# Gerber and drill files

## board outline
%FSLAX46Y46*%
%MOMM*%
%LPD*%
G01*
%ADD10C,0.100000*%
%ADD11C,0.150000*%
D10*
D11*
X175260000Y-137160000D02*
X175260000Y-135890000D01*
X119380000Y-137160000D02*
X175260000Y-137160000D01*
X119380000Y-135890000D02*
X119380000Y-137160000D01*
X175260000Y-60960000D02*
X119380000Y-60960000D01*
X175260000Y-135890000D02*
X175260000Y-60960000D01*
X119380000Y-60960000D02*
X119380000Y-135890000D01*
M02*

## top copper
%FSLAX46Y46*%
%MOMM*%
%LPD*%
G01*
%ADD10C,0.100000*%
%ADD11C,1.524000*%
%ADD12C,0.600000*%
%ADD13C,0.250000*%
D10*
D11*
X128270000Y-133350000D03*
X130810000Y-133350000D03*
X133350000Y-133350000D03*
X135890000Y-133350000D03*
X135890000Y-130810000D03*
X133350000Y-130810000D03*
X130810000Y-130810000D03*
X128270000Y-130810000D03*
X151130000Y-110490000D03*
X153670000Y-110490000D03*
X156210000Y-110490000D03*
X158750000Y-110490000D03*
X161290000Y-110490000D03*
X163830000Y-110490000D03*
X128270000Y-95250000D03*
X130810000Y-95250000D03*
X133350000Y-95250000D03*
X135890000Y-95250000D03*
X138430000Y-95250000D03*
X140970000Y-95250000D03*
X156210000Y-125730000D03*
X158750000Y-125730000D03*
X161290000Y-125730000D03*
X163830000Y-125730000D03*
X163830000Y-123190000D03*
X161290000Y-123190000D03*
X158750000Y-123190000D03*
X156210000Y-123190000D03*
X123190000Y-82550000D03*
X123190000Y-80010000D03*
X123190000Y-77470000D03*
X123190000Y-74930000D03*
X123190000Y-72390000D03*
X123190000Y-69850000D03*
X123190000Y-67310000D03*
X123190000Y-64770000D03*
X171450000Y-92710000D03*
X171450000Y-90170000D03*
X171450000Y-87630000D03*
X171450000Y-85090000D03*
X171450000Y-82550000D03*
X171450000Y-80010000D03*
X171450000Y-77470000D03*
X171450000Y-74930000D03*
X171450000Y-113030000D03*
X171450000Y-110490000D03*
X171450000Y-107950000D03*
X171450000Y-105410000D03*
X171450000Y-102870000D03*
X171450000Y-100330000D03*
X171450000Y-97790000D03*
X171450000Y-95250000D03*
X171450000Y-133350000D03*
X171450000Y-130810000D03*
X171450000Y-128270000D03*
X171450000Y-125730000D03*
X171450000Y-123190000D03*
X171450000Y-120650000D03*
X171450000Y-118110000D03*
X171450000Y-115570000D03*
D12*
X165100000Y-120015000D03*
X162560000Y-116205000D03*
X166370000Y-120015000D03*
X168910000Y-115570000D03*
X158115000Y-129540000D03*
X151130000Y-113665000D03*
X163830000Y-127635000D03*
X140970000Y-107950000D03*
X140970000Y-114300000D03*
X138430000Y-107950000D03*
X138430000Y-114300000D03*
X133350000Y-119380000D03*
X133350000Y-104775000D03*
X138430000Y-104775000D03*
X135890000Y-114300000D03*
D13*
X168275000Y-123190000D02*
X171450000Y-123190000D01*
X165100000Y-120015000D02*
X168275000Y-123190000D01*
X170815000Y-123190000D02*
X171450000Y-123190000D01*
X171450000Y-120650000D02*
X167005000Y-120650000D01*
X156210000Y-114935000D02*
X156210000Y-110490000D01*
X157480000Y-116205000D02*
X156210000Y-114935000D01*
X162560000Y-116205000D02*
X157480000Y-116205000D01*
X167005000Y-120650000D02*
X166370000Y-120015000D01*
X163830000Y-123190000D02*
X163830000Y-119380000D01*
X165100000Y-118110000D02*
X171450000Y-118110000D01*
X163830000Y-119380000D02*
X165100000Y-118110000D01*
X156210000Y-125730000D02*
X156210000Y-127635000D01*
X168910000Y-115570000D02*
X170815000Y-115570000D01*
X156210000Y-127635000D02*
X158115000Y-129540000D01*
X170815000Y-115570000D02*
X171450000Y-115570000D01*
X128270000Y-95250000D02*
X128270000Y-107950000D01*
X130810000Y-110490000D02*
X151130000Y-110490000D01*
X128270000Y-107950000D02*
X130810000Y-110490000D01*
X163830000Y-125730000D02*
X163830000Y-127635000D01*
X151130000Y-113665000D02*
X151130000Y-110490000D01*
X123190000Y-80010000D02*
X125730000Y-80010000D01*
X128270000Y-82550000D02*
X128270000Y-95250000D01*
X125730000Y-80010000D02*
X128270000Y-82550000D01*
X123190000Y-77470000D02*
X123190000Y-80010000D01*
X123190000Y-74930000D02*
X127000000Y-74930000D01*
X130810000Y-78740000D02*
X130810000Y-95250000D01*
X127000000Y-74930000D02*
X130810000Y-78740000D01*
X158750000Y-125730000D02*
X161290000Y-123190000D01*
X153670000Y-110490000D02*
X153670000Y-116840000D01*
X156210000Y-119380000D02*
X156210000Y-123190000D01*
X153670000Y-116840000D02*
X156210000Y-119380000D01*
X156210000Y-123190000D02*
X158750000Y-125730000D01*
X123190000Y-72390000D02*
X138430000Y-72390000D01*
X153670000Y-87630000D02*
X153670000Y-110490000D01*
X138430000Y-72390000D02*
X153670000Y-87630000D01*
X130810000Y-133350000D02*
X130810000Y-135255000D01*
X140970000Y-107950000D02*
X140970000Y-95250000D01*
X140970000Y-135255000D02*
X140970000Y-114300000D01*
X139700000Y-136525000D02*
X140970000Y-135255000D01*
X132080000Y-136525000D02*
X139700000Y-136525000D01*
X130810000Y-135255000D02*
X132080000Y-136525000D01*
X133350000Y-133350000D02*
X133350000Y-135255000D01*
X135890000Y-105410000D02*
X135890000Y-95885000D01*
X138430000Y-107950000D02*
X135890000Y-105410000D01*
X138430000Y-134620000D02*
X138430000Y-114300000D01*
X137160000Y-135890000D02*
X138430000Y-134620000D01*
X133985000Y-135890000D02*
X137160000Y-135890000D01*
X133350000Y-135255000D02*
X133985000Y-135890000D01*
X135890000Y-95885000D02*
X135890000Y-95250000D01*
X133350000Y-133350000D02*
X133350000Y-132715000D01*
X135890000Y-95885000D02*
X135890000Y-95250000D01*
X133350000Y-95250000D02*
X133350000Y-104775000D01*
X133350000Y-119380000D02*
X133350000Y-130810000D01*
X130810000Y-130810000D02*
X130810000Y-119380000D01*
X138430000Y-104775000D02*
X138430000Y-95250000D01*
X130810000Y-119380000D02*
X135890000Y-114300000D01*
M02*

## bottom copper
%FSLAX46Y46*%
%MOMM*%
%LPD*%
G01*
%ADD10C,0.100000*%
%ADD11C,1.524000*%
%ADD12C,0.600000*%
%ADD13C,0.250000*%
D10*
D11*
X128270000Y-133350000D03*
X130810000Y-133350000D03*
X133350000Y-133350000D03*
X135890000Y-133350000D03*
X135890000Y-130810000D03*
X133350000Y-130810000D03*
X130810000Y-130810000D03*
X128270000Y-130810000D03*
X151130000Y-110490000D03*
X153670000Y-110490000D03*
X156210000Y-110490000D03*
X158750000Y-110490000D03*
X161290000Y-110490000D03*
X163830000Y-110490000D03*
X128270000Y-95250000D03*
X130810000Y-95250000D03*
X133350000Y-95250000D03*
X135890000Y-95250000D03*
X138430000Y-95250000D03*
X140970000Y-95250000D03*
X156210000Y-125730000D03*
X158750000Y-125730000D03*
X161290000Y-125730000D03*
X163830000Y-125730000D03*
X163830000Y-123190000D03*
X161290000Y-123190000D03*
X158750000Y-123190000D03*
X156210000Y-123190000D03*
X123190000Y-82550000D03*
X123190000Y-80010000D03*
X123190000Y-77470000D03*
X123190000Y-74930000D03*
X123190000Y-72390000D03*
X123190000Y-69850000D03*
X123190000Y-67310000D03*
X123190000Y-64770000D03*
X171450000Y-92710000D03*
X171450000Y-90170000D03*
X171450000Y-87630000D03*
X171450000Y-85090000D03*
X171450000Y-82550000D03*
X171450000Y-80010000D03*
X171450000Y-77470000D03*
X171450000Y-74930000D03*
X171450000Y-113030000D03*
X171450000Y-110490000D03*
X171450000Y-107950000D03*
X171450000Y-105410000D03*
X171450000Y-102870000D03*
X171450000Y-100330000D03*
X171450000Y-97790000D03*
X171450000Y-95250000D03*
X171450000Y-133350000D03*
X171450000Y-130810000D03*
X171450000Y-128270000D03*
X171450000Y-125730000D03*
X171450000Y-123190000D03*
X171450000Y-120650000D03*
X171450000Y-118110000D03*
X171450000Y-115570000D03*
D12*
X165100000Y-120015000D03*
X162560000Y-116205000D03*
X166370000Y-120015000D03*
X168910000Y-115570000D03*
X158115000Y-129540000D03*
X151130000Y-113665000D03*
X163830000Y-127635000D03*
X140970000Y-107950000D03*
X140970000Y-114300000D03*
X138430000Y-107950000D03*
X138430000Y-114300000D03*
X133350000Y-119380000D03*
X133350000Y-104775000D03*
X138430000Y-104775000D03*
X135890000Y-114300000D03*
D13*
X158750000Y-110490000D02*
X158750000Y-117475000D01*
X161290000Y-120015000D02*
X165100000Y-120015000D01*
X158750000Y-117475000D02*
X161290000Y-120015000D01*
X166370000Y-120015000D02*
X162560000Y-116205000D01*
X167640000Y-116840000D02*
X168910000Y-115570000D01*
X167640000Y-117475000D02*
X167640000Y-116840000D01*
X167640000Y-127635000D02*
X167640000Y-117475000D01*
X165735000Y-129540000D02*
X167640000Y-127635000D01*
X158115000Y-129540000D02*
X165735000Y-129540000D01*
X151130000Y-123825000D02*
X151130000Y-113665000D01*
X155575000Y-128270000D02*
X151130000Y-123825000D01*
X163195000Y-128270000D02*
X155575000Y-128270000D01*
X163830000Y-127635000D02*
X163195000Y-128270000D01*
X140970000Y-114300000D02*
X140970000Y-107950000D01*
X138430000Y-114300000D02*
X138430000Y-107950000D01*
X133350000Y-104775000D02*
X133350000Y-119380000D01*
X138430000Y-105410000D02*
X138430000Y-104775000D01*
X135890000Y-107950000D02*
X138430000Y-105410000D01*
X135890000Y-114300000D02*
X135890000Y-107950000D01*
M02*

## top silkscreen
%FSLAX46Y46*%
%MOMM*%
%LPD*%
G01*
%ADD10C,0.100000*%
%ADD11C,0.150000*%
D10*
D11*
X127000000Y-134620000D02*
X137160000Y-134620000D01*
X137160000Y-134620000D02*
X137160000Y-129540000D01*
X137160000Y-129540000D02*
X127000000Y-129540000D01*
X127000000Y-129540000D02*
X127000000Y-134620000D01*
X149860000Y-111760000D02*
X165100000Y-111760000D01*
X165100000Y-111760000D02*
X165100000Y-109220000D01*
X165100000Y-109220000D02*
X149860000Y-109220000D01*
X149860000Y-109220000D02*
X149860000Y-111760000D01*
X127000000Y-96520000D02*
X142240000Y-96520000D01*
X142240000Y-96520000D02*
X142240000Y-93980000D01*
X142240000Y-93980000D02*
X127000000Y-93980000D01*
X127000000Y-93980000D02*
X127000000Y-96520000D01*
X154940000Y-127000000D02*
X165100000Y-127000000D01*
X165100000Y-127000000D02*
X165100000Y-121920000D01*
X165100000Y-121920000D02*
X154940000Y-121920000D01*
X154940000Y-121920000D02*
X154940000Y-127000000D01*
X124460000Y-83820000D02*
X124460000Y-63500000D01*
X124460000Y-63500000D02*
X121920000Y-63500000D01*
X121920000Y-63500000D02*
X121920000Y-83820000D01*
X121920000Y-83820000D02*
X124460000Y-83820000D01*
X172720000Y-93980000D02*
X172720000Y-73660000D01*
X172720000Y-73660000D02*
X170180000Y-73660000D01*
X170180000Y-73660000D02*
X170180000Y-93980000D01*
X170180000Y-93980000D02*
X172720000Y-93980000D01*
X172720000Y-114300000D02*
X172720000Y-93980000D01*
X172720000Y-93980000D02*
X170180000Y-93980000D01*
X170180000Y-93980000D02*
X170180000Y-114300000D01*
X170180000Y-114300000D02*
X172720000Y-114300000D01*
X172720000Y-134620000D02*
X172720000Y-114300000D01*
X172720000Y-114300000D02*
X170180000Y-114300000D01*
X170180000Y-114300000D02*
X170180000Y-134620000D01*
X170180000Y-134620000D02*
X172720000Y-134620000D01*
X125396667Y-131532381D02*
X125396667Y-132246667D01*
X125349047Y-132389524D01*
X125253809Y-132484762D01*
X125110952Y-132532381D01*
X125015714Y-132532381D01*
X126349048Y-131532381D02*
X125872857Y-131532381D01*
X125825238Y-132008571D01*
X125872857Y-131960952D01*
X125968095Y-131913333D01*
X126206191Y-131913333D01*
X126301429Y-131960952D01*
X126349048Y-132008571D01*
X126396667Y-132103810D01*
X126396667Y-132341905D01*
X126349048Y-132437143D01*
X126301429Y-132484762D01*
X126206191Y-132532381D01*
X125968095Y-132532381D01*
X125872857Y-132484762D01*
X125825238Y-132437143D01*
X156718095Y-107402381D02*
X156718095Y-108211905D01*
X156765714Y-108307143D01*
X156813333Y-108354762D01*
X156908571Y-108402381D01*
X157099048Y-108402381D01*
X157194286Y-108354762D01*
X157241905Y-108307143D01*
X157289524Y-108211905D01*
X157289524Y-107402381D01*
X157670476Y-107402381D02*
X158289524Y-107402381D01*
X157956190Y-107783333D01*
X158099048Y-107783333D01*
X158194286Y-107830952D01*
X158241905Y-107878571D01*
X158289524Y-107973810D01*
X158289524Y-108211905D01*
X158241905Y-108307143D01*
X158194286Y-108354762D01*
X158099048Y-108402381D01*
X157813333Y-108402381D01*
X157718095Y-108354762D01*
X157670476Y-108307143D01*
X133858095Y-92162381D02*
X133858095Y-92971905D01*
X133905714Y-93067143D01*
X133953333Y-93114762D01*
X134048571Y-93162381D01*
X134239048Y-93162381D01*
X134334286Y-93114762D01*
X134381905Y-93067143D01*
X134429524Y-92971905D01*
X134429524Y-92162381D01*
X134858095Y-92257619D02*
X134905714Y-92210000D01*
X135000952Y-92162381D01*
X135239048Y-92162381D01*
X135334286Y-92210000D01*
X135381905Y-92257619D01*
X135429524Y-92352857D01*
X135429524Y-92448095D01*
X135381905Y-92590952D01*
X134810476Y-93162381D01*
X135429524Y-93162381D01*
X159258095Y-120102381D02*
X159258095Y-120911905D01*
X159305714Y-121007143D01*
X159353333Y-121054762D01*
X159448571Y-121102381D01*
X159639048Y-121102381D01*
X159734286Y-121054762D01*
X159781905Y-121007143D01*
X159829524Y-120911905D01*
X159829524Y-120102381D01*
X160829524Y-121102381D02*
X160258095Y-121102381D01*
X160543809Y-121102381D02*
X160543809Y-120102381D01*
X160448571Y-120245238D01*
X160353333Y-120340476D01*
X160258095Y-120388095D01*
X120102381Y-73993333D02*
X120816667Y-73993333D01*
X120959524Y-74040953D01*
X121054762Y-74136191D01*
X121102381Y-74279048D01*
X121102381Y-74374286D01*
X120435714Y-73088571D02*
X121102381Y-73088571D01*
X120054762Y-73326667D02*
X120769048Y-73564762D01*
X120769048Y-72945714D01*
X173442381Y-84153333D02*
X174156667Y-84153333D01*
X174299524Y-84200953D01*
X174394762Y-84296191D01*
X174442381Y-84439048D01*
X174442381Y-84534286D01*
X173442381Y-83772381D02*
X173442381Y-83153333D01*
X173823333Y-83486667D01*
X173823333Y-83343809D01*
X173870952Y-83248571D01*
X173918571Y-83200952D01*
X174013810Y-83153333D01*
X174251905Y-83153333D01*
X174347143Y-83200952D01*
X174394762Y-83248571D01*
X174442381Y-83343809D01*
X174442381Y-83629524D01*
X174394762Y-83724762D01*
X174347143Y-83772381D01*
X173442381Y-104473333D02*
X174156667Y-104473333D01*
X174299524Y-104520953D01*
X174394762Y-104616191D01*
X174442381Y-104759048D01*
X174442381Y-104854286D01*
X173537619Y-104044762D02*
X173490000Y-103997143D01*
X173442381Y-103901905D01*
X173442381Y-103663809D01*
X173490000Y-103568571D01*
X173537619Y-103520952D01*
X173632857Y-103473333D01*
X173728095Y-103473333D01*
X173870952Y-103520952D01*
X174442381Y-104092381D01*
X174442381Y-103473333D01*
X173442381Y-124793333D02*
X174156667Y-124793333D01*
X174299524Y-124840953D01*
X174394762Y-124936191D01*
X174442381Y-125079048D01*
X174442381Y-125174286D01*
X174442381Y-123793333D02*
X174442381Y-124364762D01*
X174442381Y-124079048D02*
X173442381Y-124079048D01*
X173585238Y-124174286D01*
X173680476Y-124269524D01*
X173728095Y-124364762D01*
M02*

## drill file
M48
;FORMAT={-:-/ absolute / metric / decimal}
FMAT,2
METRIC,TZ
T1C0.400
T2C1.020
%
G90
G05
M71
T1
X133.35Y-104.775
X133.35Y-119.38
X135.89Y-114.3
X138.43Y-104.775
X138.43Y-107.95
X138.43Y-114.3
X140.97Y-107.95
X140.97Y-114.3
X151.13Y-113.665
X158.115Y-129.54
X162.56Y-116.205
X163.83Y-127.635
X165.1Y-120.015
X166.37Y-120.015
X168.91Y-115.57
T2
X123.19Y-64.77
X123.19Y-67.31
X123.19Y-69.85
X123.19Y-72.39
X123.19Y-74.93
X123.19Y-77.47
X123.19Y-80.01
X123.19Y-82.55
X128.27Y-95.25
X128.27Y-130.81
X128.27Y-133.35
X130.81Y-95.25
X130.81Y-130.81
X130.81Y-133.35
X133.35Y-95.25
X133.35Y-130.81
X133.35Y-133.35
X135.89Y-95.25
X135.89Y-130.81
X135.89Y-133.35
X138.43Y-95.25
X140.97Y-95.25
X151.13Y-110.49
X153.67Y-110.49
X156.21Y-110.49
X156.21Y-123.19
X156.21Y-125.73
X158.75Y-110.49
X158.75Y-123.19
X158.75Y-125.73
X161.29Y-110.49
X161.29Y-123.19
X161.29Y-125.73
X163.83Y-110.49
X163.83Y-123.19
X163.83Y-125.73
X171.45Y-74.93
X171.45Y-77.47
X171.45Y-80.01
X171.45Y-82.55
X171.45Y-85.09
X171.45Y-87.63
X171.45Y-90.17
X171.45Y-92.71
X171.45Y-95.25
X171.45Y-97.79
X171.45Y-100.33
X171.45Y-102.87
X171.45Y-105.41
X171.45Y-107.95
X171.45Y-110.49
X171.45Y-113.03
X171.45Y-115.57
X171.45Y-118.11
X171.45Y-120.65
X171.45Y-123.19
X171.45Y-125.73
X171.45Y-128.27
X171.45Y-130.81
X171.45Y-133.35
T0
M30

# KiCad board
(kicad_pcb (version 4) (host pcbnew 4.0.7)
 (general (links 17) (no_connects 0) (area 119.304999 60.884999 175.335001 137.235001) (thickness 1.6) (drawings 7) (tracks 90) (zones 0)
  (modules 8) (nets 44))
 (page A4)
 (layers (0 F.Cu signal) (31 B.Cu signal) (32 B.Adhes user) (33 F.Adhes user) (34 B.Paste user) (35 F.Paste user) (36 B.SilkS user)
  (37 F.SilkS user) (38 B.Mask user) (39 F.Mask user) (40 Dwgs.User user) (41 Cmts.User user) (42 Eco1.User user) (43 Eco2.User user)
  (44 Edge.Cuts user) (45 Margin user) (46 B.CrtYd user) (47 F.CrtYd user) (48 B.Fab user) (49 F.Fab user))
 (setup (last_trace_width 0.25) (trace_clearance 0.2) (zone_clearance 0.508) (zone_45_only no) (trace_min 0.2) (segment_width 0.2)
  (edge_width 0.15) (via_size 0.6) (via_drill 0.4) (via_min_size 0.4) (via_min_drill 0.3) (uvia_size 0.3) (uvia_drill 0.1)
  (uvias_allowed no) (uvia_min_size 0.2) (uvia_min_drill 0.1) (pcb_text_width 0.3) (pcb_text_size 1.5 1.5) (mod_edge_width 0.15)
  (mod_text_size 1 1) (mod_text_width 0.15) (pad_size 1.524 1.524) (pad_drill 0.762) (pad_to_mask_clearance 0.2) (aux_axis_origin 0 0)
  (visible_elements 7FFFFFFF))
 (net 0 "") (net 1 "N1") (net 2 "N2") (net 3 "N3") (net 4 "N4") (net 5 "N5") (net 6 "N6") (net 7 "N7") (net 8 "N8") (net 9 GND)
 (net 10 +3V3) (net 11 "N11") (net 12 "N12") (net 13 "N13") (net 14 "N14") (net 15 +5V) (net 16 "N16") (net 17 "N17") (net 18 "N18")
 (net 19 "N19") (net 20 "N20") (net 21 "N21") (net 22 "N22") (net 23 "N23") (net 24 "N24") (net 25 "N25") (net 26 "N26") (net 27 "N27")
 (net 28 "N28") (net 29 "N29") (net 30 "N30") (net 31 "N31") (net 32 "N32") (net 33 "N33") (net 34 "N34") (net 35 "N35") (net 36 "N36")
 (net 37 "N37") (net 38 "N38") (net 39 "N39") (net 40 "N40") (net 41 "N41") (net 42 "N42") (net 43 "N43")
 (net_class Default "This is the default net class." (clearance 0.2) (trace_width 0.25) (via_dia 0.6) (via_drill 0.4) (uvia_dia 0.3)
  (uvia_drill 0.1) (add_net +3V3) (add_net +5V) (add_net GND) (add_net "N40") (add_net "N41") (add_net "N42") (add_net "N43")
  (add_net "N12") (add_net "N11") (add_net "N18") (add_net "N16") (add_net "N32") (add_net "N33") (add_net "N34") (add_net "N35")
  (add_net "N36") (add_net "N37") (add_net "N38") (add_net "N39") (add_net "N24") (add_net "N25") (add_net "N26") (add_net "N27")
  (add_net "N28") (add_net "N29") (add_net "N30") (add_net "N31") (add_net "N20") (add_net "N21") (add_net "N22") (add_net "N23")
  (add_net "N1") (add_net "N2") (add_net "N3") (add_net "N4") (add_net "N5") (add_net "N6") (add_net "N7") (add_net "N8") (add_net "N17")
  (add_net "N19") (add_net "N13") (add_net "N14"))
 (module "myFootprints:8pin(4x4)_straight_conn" (layer F.Cu) (at 132.08 132.08)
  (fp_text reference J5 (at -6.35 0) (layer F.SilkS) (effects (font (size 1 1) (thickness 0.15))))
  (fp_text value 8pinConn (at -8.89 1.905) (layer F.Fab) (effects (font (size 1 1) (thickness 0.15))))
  (fp_line (start -5.08 2.54) (end 5.08 2.54) (layer F.SilkS) (width 0.15))
  (fp_line (start 5.08 2.54) (end 5.08 -2.54) (layer F.SilkS) (width 0.15))
  (fp_line (start 5.08 -2.54) (end -5.08 -2.54) (layer F.SilkS) (width 0.15))
  (fp_line (start -5.08 -2.54) (end -5.08 2.54) (layer F.SilkS) (width 0.15))
  (pad 1 thru_hole circle (at -3.81 1.27) (size 1.524 1.524) (drill 1.02) (layers *.Cu *.Mask) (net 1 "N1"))
  (pad 2 thru_hole circle (at -1.27 1.27) (size 1.524 1.524) (drill 1.02) (layers *.Cu *.Mask) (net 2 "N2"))
  (pad 3 thru_hole circle (at 1.27 1.27) (size 1.524 1.524) (drill 1.02) (layers *.Cu *.Mask) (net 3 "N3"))
  (pad 4 thru_hole circle (at 3.81 1.27) (size 1.524 1.524) (drill 1.02) (layers *.Cu *.Mask) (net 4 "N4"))
  (pad 5 thru_hole circle (at 3.81 -1.27) (size 1.524 1.524) (drill 1.02) (layers *.Cu *.Mask) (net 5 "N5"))
  (pad 6 thru_hole circle (at 1.27 -1.27) (size 1.524 1.524) (drill 1.02) (layers *.Cu *.Mask) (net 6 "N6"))
  (pad 7 thru_hole circle (at -1.27 -1.27) (size 1.524 1.524) (drill 1.02) (layers *.Cu *.Mask) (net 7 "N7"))
  (pad 8 thru_hole circle (at -3.81 -1.27) (size 1.524 1.524) (drill 1.02) (layers *.Cu *.Mask) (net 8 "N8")))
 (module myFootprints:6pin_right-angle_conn (layer F.Cu) (at 157.48 110.49)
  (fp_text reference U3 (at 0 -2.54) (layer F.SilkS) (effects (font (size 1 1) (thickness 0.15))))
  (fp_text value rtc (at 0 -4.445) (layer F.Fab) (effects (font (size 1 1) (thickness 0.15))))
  (fp_line (start -7.62 1.27) (end 7.62 1.27) (layer F.SilkS) (width 0.15))
  (fp_line (start 7.62 1.27) (end 7.62 -1.27) (layer F.SilkS) (width 0.15))
  (fp_line (start 7.62 -1.27) (end -7.62 -1.27) (layer F.SilkS) (width 0.15))
  (fp_line (start -7.62 -1.27) (end -7.62 1.27) (layer F.SilkS) (width 0.15))
  (pad 1 thru_hole circle (at -6.35 0) (size 1.524 1.524) (drill 1.02) (layers *.Cu *.Mask) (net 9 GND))
  (pad 2 thru_hole circle (at -3.81 0) (size 1.524 1.524) (drill 1.02) (layers *.Cu *.Mask) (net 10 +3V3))
  (pad 3 thru_hole circle (at -1.27 0) (size 1.524 1.524) (drill 1.02) (layers *.Cu *.Mask) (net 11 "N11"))
  (pad 4 thru_hole circle (at 1.27 0) (size 1.524 1.524) (drill 1.02) (layers *.Cu *.Mask) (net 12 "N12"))
  (pad 5 thru_hole circle (at 3.81 0) (size 1.524 1.524) (drill 1.02) (layers *.Cu *.Mask) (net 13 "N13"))
  (pad 6 thru_hole circle (at 6.35 0) (size 1.524 1.524) (drill 1.02) (layers *.Cu *.Mask) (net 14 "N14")))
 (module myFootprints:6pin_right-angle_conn (layer F.Cu) (at 134.62 95.25)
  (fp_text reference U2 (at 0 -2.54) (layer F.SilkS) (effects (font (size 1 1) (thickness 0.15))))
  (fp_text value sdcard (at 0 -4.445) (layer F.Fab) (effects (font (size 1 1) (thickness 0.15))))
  (fp_line (start -7.62 1.27) (end 7.62 1.27) (layer F.SilkS) (width 0.15))
  (fp_line (start 7.62 1.27) (end 7.62 -1.27) (layer F.SilkS) (width 0.15))
  (fp_line (start 7.62 -1.27) (end -7.62 -1.27) (layer F.SilkS) (width 0.15))
  (fp_line (start -7.62 -1.27) (end -7.62 1.27) (layer F.SilkS) (width 0.15))
  (pad 1 thru_hole circle (at -6.35 0) (size 1.524 1.524) (drill 1.02) (layers *.Cu *.Mask) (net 9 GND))
  (pad 2 thru_hole circle (at -3.81 0) (size 1.524 1.524) (drill 1.02) (layers *.Cu *.Mask) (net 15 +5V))
  (pad 3 thru_hole circle (at -1.27 0) (size 1.524 1.524) (drill 1.02) (layers *.Cu *.Mask) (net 6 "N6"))
  (pad 4 thru_hole circle (at 1.27 0) (size 1.524 1.524) (drill 1.02) (layers *.Cu *.Mask) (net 3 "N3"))
  (pad 5 thru_hole circle (at 3.81 0) (size 1.524 1.524) (drill 1.02) (layers *.Cu *.Mask) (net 7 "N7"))
  (pad 6 thru_hole circle (at 6.35 0) (size 1.524 1.524) (drill 1.02) (layers *.Cu *.Mask) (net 2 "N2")))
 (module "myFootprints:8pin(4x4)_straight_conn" (layer F.Cu) (at 160.02 124.46)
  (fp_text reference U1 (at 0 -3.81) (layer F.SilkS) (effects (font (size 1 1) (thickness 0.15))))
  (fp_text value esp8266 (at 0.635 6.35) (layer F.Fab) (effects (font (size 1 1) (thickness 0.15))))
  (fp_line (start -5.08 2.54) (end 5.08 2.54) (layer F.SilkS) (width 0.15))
  (fp_line (start 5.08 2.54) (end 5.08 -2.54) (layer F.SilkS) (width 0.15))
  (fp_line (start 5.08 -2.54) (end -5.08 -2.54) (layer F.SilkS) (width 0.15))
  (fp_line (start -5.08 -2.54) (end -5.08 2.54) (layer F.SilkS) (width 0.15))
  (pad 1 thru_hole circle (at -3.81 1.27) (size 1.524 1.524) (drill 1.02) (layers *.Cu *.Mask) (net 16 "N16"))
  (pad 2 thru_hole circle (at -1.27 1.27) (size 1.524 1.524) (drill 1.02) (layers *.Cu *.Mask) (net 10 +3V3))
  (pad 3 thru_hole circle (at 1.27 1.27) (size 1.524 1.524) (drill 1.02) (layers *.Cu *.Mask) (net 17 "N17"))
  (pad 4 thru_hole circle (at 3.81 1.27) (size 1.524 1.524) (drill 1.02) (layers *.Cu *.Mask) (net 9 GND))
  (pad 5 thru_hole circle (at 3.81 -1.27) (size 1.524 1.524) (drill 1.02) (layers *.Cu *.Mask) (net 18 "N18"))
  (pad 6 thru_hole circle (at 1.27 -1.27) (size 1.524 1.524) (drill 1.02) (layers *.Cu *.Mask) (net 10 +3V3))
  (pad 7 thru_hole circle (at -1.27 -1.27) (size 1.524 1.524) (drill 1.02) (layers *.Cu *.Mask) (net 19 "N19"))
  (pad 8 thru_hole circle (at -3.81 -1.27) (size 1.524 1.524) (drill 1.02) (layers *.Cu *.Mask) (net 10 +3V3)))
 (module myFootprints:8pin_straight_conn (layer F.Cu) (at 123.19 73.66 90)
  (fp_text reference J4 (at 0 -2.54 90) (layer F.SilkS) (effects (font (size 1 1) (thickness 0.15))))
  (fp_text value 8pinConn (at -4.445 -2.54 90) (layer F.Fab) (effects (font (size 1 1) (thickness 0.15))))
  (fp_line (start -10.16 1.27) (end 10.16 1.27) (layer F.SilkS) (width 0.15))
  (fp_line (start 10.16 1.27) (end 10.16 -1.27) (layer F.SilkS) (width 0.15))
  (fp_line (start 10.16 -1.27) (end -10.16 -1.27) (layer F.SilkS) (width 0.15))
  (fp_line (start -10.16 -1.27) (end -10.16 1.27) (layer F.SilkS) (width 0.15))
  (pad 1 thru_hole circle (at -8.89 0 90) (size 1.524 1.524) (drill 1.02) (layers *.Cu *.Mask) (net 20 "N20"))
  (pad 2 thru_hole circle (at -6.35 0 90) (size 1.524 1.524) (drill 1.02) (layers *.Cu *.Mask) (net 9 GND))
  (pad 3 thru_hole circle (at -3.81 0 90) (size 1.524 1.524) (drill 1.02) (layers *.Cu *.Mask) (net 9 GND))
  (pad 4 thru_hole circle (at -1.27 0 90) (size 1.524 1.524) (drill 1.02) (layers *.Cu *.Mask) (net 15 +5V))
  (pad 5 thru_hole circle (at 1.27 0 90) (size 1.524 1.524) (drill 1.02) (layers *.Cu *.Mask) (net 10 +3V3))
  (pad 6 thru_hole circle (at 3.81 0 90) (size 1.524 1.524) (drill 1.02) (layers *.Cu *.Mask) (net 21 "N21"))
  (pad 7 thru_hole circle (at 6.35 0 90) (size 1.524 1.524) (drill 1.02) (layers *.Cu *.Mask) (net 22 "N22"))
  (pad 8 thru_hole circle (at 8.89 0 90) (size 1.524 1.524) (drill 1.02) (layers *.Cu *.Mask) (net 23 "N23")))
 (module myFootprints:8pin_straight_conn (layer F.Cu) (at 171.45 83.82 90)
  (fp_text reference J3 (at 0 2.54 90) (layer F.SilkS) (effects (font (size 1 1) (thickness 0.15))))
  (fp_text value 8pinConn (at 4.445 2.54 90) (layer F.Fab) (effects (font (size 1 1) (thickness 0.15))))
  (fp_line (start -10.16 1.27) (end 10.16 1.27) (layer F.SilkS) (width 0.15))
  (fp_line (start 10.16 1.27) (end 10.16 -1.27) (layer F.SilkS) (width 0.15))
  (fp_line (start 10.16 -1.27) (end -10.16 -1.27) (layer F.SilkS) (width 0.15))
  (fp_line (start -10.16 -1.27) (end -10.16 1.27) (layer F.SilkS) (width 0.15))
  (pad 1 thru_hole circle (at -8.89 0 90) (size 1.524 1.524) (drill 1.02) (layers *.Cu *.Mask) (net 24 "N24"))
  (pad 2 thru_hole circle (at -6.35 0 90) (size 1.524 1.524) (drill 1.02) (layers *.Cu *.Mask) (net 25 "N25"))
  (pad 3 thru_hole circle (at -3.81 0 90) (size 1.524 1.524) (drill 1.02) (layers *.Cu *.Mask) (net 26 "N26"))
  (pad 4 thru_hole circle (at -1.27 0 90) (size 1.524 1.524) (drill 1.02) (layers *.Cu *.Mask) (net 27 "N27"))
  (pad 5 thru_hole circle (at 1.27 0 90) (size 1.524 1.524) (drill 1.02) (layers *.Cu *.Mask) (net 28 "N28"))
  (pad 6 thru_hole circle (at 3.81 0 90) (size 1.524 1.524) (drill 1.02) (layers *.Cu *.Mask) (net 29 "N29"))
  (pad 7 thru_hole circle (at 6.35 0 90) (size 1.524 1.524) (drill 1.02) (layers *.Cu *.Mask) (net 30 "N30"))
  (pad 8 thru_hole circle (at 8.89 0 90) (size 1.524 1.524) (drill 1.02) (layers *.Cu *.Mask) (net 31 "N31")))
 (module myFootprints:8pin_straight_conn (layer F.Cu) (at 171.45 104.14 90)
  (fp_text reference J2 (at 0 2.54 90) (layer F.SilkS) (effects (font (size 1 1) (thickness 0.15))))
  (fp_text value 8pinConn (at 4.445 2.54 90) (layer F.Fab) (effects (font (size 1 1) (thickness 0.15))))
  (fp_line (start -10.16 1.27) (end 10.16 1.27) (layer F.SilkS) (width 0.15))
  (fp_line (start 10.16 1.27) (end 10.16 -1.27) (layer F.SilkS) (width 0.15))
  (fp_line (start 10.16 -1.27) (end -10.16 -1.27) (layer F.SilkS) (width 0.15))
  (fp_line (start -10.16 -1.27) (end -10.16 1.27) (layer F.SilkS) (width 0.15))
  (pad 1 thru_hole circle (at -8.89 0 90) (size 1.524 1.524) (drill 1.02) (layers *.Cu *.Mask) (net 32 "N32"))
  (pad 2 thru_hole circle (at -6.35 0 90) (size 1.524 1.524) (drill 1.02) (layers *.Cu *.Mask) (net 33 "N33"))
  (pad 3 thru_hole circle (at -3.81 0 90) (size 1.524 1.524) (drill 1.02) (layers *.Cu *.Mask) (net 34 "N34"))
  (pad 4 thru_hole circle (at -1.27 0 90) (size 1.524 1.524) (drill 1.02) (layers *.Cu *.Mask) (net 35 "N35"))
  (pad 5 thru_hole circle (at 1.27 0 90) (size 1.524 1.524) (drill 1.02) (layers *.Cu *.Mask) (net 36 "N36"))
  (pad 6 thru_hole circle (at 3.81 0 90) (size 1.524 1.524) (drill 1.02) (layers *.Cu *.Mask) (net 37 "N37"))
  (pad 7 thru_hole circle (at 6.35 0 90) (size 1.524 1.524) (drill 1.02) (layers *.Cu *.Mask) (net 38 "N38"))
  (pad 8 thru_hole circle (at 8.89 0 90) (size 1.524 1.524) (drill 1.02) (layers *.Cu *.Mask) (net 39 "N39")))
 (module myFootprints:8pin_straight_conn (layer F.Cu) (at 171.45 124.46 90)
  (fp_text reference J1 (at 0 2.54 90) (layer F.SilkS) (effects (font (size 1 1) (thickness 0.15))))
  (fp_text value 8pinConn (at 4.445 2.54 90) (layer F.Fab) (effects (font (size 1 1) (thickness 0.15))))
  (fp_line (start -10.16 1.27) (end 10.16 1.27) (layer F.SilkS) (width 0.15))
  (fp_line (start 10.16 1.27) (end 10.16 -1.27) (layer F.SilkS) (width 0.15))
  (fp_line (start 10.16 -1.27) (end -10.16 -1.27) (layer F.SilkS) (width 0.15))
  (fp_line (start -10.16 -1.27) (end -10.16 1.27) (layer F.SilkS) (width 0.15))
  (pad 1 thru_hole circle (at -8.89 0 90) (size 1.524 1.524) (drill 1.02) (layers *.Cu *.Mask) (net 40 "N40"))
  (pad 2 thru_hole circle (at -6.35 0 90) (size 1.524 1.524) (drill 1.02) (layers *.Cu *.Mask) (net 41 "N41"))
  (pad 3 thru_hole circle (at -3.81 0 90) (size 1.524 1.524) (drill 1.02) (layers *.Cu *.Mask) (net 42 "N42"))
  (pad 4 thru_hole circle (at -1.27 0 90) (size 1.524 1.524) (drill 1.02) (layers *.Cu *.Mask) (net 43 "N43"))
  (pad 5 thru_hole circle (at 1.27 0 90) (size 1.524 1.524) (drill 1.02) (layers *.Cu *.Mask) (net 12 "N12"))
  (pad 6 thru_hole circle (at 3.81 0 90) (size 1.524 1.524) (drill 1.02) (layers *.Cu *.Mask) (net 11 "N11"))
  (pad 7 thru_hole circle (at 6.35 0 90) (size 1.524 1.524) (drill 1.02) (layers *.Cu *.Mask) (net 18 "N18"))
  (pad 8 thru_hole circle (at 8.89 0 90) (size 1.524 1.524) (drill 1.02) (layers *.Cu *.Mask) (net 16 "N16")))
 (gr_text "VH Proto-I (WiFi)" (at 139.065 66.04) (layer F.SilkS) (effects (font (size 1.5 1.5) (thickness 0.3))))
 (gr_line (start 175.26 137.16) (end 175.26 135.89) (angle 90) (layer Edge.Cuts) (width 0.15))
 (gr_line (start 119.38 137.16) (end 175.26 137.16) (angle 90) (layer Edge.Cuts) (width 0.15))
 (gr_line (start 119.38 135.89) (end 119.38 137.16) (angle 90) (layer Edge.Cuts) (width 0.15))
 (gr_line (start 175.26 60.96) (end 119.38 60.96) (angle 90) (layer Edge.Cuts) (width 0.15))
 (gr_line (start 175.26 135.89) (end 175.26 60.96) (angle 90) (layer Edge.Cuts) (width 0.15))
 (gr_line (start 119.38 60.96) (end 119.38 135.89) (angle 90) (layer Edge.Cuts) (width 0.15))
 (segment (start 158.75 110.49) (end 158.75 117.475) (width 0.25) (layer B.Cu) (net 12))
 (segment (start 168.275 123.19) (end 171.45 123.19) (width 0.25) (layer F.Cu) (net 12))
 (segment (start 165.1 120.015) (end 168.275 123.19) (width 0.25) (layer F.Cu) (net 12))
 (via (at 165.1 120.015) (size 0.6) (drill 0.4) (layers F.Cu B.Cu) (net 12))
 (segment (start 161.29 120.015) (end 165.1 120.015) (width 0.25) (layer B.Cu) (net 12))
 (segment (start 158.75 117.475) (end 161.29 120.015) (width 0.25) (layer B.Cu) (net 12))
 (segment (start 170.815 123.19) (end 171.45 123.19) (width 0.25) (layer F.Cu) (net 12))
 (segment (start 171.45 120.65) (end 167.005 120.65) (width 0.25) (layer F.Cu) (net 11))
 (segment (start 156.21 114.935) (end 156.21 110.49) (width 0.25) (layer F.Cu) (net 11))
 (segment (start 157.48 116.205) (end 156.21 114.935) (width 0.25) (layer F.Cu) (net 11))
 (segment (start 162.56 116.205) (end 157.48 116.205) (width 0.25) (layer F.Cu) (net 11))
 (via (at 162.56 116.205) (size 0.6) (drill 0.4) (layers F.Cu B.Cu) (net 11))
 (segment (start 166.37 120.015) (end 162.56 116.205) (width 0.25) (layer B.Cu) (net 11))
 (via (at 166.37 120.015) (size 0.6) (drill 0.4) (layers F.Cu B.Cu) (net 11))
 (segment (start 167.005 120.65) (end 166.37 120.015) (width 0.25) (layer F.Cu) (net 11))
 (segment (start 163.83 123.19) (end 163.83 119.38) (width 0.25) (layer F.Cu) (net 18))
 (segment (start 165.1 118.11) (end 171.45 118.11) (width 0.25) (layer F.Cu) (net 18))
 (segment (start 163.83 119.38) (end 165.1 118.11) (width 0.25) (layer F.Cu) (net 18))
 (segment (start 156.21 125.73) (end 156.21 127.635) (width 0.25) (layer F.Cu) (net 16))
 (segment (start 168.91 115.57) (end 170.815 115.57) (width 0.25) (layer F.Cu) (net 16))
 (via (at 168.91 115.57) (size 0.6) (drill 0.4) (layers F.Cu B.Cu) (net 16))
 (segment (start 167.64 116.84) (end 168.91 115.57) (width 0.25) (layer B.Cu) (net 16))
 (segment (start 167.64 117.475) (end 167.64 116.84) (width 0.25) (layer B.Cu) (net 16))
 (segment (start 167.64 127.635) (end 167.64 117.475) (width 0.25) (layer B.Cu) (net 16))
 (segment (start 165.735 129.54) (end 167.64 127.635) (width 0.25) (layer B.Cu) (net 16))
 (segment (start 158.115 129.54) (end 165.735 129.54) (width 0.25) (layer B.Cu) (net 16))
 (via (at 158.115 129.54) (size 0.6) (drill 0.4) (layers F.Cu B.Cu) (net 16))
 (segment (start 156.21 127.635) (end 158.115 129.54) (width 0.25) (layer F.Cu) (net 16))
 (segment (start 170.815 115.57) (end 171.45 115.57) (width 0.25) (layer F.Cu) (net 16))
 (segment (start 128.27 95.25) (end 128.27 107.95) (width 0.25) (layer F.Cu) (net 9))
 (segment (start 130.81 110.49) (end 151.13 110.49) (width 0.25) (layer F.Cu) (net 9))
 (segment (start 128.27 107.95) (end 130.81 110.49) (width 0.25) (layer F.Cu) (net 9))
 (segment (start 163.83 125.73) (end 163.83 127.635) (width 0.25) (layer F.Cu) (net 9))
 (segment (start 151.13 113.665) (end 151.13 110.49) (width 0.25) (layer F.Cu) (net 9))
 (via (at 151.13 113.665) (size 0.6) (drill 0.4) (layers F.Cu B.Cu) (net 9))
 (segment (start 151.13 123.825) (end 151.13 113.665) (width 0.25) (layer B.Cu) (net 9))
 (segment (start 155.575 128.27) (end 151.13 123.825) (width 0.25) (layer B.Cu) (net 9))
 (segment (start 163.195 128.27) (end 155.575 128.27) (width 0.25) (layer B.Cu) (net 9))
 (segment (start 163.83 127.635) (end 163.195 128.27) (width 0.25) (layer B.Cu) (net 9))
 (via (at 163.83 127.635) (size 0.6) (drill 0.4) (layers F.Cu B.Cu) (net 9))
 (segment (start 123.19 80.01) (end 125.73 80.01) (width 0.25) (layer F.Cu) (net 9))
 (segment (start 128.27 82.55) (end 128.27 95.25) (width 0.25) (layer F.Cu) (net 9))
 (segment (start 125.73 80.01) (end 128.27 82.55) (width 0.25) (layer F.Cu) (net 9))
 (segment (start 123.19 77.47) (end 123.19 80.01) (width 0.25) (layer F.Cu) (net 9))
 (segment (start 123.19 74.93) (end 127 74.93) (width 0.25) (layer F.Cu) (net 15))
 (segment (start 130.81 78.74) (end 130.81 95.25) (width 0.25) (layer F.Cu) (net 15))
 (segment (start 127 74.93) (end 130.81 78.74) (width 0.25) (layer F.Cu) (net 15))
 (segment (start 158.75 125.73) (end 161.29 123.19) (width 0.25) (layer F.Cu) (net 10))
 (segment (start 153.67 110.49) (end 153.67 116.84) (width 0.25) (layer F.Cu) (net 10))
 (segment (start 156.21 119.38) (end 156.21 123.19) (width 0.25) (layer F.Cu) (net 10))
 (segment (start 153.67 116.84) (end 156.21 119.38) (width 0.25) (layer F.Cu) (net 10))
 (segment (start 156.21 123.19) (end 158.75 125.73) (width 0.25) (layer F.Cu) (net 10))
 (segment (start 123.19 72.39) (end 138.43 72.39) (width 0.25) (layer F.Cu) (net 10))
 (segment (start 153.67 87.63) (end 153.67 110.49) (width 0.25) (layer F.Cu) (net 10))
 (segment (start 138.43 72.39) (end 153.67 87.63) (width 0.25) (layer F.Cu) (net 10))
 (segment (start 130.81 133.35) (end 130.81 135.255) (width 0.25) (layer F.Cu) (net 2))
 (segment (start 140.97 107.95) (end 140.97 95.25) (width 0.25) (layer F.Cu) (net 2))
 (via (at 140.97 107.95) (size 0.6) (drill 0.4) (layers F.Cu B.Cu) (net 2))
 (segment (start 140.97 114.3) (end 140.97 107.95) (width 0.25) (layer B.Cu) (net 2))
 (via (at 140.97 114.3) (size 0.6) (drill 0.4) (layers F.Cu B.Cu) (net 2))
 (segment (start 140.97 135.255) (end 140.97 114.3) (width 0.25) (layer F.Cu) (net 2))
 (segment (start 139.7 136.525) (end 140.97 135.255) (width 0.25) (layer F.Cu) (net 2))
 (segment (start 132.08 136.525) (end 139.7 136.525) (width 0.25) (layer F.Cu) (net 2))
 (segment (start 130.81 135.255) (end 132.08 136.525) (width 0.25) (layer F.Cu) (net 2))
 (segment (start 133.35 133.35) (end 133.35 135.255) (width 0.25) (layer F.Cu) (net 3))
 (segment (start 135.89 105.41) (end 135.89 95.885) (width 0.25) (layer F.Cu) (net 3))
 (segment (start 138.43 107.95) (end 135.89 105.41) (width 0.25) (layer F.Cu) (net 3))
 (via (at 138.43 107.95) (size 0.6) (drill 0.4) (layers F.Cu B.Cu) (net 3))
 (segment (start 138.43 114.3) (end 138.43 107.95) (width 0.25) (layer B.Cu) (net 3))
 (via (at 138.43 114.3) (size 0.6) (drill 0.4) (layers F.Cu B.Cu) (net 3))
 (segment (start 138.43 134.62) (end 138.43 114.3) (width 0.25) (layer F.Cu) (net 3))
 (segment (start 137.16 135.89) (end 138.43 134.62) (width 0.25) (layer F.Cu) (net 3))
 (segment (start 133.985 135.89) (end 137.16 135.89) (width 0.25) (layer F.Cu) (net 3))
 (segment (start 133.35 135.255) (end 133.985 135.89) (width 0.25) (layer F.Cu) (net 3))
 (segment (start 135.89 95.885) (end 135.89 95.25) (width 0.25) (layer F.Cu) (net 3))
 (segment (start 133.35 133.35) (end 133.35 132.715) (width 0.25) (layer F.Cu) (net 3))
 (segment (start 135.89 95.885) (end 135.89 95.25) (width 0.25) (layer F.Cu) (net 3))
 (segment (start 133.35 95.25) (end 133.35 104.775) (width 0.25) (layer F.Cu) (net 6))
 (segment (start 133.35 119.38) (end 133.35 130.81) (width 0.25) (layer F.Cu) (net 6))
 (via (at 133.35 119.38) (size 0.6) (drill 0.4) (layers F.Cu B.Cu) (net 6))
 (segment (start 133.35 104.775) (end 133.35 119.38) (width 0.25) (layer B.Cu) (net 6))
 (via (at 133.35 104.775) (size 0.6) (drill 0.4) (layers F.Cu B.Cu) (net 6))
 (segment (start 130.81 130.81) (end 130.81 119.38) (width 0.25) (layer F.Cu) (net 7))
 (segment (start 138.43 104.775) (end 138.43 95.25) (width 0.25) (layer F.Cu) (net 7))
 (via (at 138.43 104.775) (size 0.6) (drill 0.4) (layers F.Cu B.Cu) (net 7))
 (segment (start 138.43 105.41) (end 138.43 104.775) (width 0.25) (layer B.Cu) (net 7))
 (segment (start 135.89 107.95) (end 138.43 105.41) (width 0.25) (layer B.Cu) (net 7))
 (segment (start 135.89 114.3) (end 135.89 107.95) (width 0.25) (layer B.Cu) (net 7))
 (via (at 135.89 114.3) (size 0.6) (drill 0.4) (layers F.Cu B.Cu) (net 7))
 (segment (start 130.81 119.38) (end 135.89 114.3) (width 0.25) (layer F.Cu) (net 7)))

